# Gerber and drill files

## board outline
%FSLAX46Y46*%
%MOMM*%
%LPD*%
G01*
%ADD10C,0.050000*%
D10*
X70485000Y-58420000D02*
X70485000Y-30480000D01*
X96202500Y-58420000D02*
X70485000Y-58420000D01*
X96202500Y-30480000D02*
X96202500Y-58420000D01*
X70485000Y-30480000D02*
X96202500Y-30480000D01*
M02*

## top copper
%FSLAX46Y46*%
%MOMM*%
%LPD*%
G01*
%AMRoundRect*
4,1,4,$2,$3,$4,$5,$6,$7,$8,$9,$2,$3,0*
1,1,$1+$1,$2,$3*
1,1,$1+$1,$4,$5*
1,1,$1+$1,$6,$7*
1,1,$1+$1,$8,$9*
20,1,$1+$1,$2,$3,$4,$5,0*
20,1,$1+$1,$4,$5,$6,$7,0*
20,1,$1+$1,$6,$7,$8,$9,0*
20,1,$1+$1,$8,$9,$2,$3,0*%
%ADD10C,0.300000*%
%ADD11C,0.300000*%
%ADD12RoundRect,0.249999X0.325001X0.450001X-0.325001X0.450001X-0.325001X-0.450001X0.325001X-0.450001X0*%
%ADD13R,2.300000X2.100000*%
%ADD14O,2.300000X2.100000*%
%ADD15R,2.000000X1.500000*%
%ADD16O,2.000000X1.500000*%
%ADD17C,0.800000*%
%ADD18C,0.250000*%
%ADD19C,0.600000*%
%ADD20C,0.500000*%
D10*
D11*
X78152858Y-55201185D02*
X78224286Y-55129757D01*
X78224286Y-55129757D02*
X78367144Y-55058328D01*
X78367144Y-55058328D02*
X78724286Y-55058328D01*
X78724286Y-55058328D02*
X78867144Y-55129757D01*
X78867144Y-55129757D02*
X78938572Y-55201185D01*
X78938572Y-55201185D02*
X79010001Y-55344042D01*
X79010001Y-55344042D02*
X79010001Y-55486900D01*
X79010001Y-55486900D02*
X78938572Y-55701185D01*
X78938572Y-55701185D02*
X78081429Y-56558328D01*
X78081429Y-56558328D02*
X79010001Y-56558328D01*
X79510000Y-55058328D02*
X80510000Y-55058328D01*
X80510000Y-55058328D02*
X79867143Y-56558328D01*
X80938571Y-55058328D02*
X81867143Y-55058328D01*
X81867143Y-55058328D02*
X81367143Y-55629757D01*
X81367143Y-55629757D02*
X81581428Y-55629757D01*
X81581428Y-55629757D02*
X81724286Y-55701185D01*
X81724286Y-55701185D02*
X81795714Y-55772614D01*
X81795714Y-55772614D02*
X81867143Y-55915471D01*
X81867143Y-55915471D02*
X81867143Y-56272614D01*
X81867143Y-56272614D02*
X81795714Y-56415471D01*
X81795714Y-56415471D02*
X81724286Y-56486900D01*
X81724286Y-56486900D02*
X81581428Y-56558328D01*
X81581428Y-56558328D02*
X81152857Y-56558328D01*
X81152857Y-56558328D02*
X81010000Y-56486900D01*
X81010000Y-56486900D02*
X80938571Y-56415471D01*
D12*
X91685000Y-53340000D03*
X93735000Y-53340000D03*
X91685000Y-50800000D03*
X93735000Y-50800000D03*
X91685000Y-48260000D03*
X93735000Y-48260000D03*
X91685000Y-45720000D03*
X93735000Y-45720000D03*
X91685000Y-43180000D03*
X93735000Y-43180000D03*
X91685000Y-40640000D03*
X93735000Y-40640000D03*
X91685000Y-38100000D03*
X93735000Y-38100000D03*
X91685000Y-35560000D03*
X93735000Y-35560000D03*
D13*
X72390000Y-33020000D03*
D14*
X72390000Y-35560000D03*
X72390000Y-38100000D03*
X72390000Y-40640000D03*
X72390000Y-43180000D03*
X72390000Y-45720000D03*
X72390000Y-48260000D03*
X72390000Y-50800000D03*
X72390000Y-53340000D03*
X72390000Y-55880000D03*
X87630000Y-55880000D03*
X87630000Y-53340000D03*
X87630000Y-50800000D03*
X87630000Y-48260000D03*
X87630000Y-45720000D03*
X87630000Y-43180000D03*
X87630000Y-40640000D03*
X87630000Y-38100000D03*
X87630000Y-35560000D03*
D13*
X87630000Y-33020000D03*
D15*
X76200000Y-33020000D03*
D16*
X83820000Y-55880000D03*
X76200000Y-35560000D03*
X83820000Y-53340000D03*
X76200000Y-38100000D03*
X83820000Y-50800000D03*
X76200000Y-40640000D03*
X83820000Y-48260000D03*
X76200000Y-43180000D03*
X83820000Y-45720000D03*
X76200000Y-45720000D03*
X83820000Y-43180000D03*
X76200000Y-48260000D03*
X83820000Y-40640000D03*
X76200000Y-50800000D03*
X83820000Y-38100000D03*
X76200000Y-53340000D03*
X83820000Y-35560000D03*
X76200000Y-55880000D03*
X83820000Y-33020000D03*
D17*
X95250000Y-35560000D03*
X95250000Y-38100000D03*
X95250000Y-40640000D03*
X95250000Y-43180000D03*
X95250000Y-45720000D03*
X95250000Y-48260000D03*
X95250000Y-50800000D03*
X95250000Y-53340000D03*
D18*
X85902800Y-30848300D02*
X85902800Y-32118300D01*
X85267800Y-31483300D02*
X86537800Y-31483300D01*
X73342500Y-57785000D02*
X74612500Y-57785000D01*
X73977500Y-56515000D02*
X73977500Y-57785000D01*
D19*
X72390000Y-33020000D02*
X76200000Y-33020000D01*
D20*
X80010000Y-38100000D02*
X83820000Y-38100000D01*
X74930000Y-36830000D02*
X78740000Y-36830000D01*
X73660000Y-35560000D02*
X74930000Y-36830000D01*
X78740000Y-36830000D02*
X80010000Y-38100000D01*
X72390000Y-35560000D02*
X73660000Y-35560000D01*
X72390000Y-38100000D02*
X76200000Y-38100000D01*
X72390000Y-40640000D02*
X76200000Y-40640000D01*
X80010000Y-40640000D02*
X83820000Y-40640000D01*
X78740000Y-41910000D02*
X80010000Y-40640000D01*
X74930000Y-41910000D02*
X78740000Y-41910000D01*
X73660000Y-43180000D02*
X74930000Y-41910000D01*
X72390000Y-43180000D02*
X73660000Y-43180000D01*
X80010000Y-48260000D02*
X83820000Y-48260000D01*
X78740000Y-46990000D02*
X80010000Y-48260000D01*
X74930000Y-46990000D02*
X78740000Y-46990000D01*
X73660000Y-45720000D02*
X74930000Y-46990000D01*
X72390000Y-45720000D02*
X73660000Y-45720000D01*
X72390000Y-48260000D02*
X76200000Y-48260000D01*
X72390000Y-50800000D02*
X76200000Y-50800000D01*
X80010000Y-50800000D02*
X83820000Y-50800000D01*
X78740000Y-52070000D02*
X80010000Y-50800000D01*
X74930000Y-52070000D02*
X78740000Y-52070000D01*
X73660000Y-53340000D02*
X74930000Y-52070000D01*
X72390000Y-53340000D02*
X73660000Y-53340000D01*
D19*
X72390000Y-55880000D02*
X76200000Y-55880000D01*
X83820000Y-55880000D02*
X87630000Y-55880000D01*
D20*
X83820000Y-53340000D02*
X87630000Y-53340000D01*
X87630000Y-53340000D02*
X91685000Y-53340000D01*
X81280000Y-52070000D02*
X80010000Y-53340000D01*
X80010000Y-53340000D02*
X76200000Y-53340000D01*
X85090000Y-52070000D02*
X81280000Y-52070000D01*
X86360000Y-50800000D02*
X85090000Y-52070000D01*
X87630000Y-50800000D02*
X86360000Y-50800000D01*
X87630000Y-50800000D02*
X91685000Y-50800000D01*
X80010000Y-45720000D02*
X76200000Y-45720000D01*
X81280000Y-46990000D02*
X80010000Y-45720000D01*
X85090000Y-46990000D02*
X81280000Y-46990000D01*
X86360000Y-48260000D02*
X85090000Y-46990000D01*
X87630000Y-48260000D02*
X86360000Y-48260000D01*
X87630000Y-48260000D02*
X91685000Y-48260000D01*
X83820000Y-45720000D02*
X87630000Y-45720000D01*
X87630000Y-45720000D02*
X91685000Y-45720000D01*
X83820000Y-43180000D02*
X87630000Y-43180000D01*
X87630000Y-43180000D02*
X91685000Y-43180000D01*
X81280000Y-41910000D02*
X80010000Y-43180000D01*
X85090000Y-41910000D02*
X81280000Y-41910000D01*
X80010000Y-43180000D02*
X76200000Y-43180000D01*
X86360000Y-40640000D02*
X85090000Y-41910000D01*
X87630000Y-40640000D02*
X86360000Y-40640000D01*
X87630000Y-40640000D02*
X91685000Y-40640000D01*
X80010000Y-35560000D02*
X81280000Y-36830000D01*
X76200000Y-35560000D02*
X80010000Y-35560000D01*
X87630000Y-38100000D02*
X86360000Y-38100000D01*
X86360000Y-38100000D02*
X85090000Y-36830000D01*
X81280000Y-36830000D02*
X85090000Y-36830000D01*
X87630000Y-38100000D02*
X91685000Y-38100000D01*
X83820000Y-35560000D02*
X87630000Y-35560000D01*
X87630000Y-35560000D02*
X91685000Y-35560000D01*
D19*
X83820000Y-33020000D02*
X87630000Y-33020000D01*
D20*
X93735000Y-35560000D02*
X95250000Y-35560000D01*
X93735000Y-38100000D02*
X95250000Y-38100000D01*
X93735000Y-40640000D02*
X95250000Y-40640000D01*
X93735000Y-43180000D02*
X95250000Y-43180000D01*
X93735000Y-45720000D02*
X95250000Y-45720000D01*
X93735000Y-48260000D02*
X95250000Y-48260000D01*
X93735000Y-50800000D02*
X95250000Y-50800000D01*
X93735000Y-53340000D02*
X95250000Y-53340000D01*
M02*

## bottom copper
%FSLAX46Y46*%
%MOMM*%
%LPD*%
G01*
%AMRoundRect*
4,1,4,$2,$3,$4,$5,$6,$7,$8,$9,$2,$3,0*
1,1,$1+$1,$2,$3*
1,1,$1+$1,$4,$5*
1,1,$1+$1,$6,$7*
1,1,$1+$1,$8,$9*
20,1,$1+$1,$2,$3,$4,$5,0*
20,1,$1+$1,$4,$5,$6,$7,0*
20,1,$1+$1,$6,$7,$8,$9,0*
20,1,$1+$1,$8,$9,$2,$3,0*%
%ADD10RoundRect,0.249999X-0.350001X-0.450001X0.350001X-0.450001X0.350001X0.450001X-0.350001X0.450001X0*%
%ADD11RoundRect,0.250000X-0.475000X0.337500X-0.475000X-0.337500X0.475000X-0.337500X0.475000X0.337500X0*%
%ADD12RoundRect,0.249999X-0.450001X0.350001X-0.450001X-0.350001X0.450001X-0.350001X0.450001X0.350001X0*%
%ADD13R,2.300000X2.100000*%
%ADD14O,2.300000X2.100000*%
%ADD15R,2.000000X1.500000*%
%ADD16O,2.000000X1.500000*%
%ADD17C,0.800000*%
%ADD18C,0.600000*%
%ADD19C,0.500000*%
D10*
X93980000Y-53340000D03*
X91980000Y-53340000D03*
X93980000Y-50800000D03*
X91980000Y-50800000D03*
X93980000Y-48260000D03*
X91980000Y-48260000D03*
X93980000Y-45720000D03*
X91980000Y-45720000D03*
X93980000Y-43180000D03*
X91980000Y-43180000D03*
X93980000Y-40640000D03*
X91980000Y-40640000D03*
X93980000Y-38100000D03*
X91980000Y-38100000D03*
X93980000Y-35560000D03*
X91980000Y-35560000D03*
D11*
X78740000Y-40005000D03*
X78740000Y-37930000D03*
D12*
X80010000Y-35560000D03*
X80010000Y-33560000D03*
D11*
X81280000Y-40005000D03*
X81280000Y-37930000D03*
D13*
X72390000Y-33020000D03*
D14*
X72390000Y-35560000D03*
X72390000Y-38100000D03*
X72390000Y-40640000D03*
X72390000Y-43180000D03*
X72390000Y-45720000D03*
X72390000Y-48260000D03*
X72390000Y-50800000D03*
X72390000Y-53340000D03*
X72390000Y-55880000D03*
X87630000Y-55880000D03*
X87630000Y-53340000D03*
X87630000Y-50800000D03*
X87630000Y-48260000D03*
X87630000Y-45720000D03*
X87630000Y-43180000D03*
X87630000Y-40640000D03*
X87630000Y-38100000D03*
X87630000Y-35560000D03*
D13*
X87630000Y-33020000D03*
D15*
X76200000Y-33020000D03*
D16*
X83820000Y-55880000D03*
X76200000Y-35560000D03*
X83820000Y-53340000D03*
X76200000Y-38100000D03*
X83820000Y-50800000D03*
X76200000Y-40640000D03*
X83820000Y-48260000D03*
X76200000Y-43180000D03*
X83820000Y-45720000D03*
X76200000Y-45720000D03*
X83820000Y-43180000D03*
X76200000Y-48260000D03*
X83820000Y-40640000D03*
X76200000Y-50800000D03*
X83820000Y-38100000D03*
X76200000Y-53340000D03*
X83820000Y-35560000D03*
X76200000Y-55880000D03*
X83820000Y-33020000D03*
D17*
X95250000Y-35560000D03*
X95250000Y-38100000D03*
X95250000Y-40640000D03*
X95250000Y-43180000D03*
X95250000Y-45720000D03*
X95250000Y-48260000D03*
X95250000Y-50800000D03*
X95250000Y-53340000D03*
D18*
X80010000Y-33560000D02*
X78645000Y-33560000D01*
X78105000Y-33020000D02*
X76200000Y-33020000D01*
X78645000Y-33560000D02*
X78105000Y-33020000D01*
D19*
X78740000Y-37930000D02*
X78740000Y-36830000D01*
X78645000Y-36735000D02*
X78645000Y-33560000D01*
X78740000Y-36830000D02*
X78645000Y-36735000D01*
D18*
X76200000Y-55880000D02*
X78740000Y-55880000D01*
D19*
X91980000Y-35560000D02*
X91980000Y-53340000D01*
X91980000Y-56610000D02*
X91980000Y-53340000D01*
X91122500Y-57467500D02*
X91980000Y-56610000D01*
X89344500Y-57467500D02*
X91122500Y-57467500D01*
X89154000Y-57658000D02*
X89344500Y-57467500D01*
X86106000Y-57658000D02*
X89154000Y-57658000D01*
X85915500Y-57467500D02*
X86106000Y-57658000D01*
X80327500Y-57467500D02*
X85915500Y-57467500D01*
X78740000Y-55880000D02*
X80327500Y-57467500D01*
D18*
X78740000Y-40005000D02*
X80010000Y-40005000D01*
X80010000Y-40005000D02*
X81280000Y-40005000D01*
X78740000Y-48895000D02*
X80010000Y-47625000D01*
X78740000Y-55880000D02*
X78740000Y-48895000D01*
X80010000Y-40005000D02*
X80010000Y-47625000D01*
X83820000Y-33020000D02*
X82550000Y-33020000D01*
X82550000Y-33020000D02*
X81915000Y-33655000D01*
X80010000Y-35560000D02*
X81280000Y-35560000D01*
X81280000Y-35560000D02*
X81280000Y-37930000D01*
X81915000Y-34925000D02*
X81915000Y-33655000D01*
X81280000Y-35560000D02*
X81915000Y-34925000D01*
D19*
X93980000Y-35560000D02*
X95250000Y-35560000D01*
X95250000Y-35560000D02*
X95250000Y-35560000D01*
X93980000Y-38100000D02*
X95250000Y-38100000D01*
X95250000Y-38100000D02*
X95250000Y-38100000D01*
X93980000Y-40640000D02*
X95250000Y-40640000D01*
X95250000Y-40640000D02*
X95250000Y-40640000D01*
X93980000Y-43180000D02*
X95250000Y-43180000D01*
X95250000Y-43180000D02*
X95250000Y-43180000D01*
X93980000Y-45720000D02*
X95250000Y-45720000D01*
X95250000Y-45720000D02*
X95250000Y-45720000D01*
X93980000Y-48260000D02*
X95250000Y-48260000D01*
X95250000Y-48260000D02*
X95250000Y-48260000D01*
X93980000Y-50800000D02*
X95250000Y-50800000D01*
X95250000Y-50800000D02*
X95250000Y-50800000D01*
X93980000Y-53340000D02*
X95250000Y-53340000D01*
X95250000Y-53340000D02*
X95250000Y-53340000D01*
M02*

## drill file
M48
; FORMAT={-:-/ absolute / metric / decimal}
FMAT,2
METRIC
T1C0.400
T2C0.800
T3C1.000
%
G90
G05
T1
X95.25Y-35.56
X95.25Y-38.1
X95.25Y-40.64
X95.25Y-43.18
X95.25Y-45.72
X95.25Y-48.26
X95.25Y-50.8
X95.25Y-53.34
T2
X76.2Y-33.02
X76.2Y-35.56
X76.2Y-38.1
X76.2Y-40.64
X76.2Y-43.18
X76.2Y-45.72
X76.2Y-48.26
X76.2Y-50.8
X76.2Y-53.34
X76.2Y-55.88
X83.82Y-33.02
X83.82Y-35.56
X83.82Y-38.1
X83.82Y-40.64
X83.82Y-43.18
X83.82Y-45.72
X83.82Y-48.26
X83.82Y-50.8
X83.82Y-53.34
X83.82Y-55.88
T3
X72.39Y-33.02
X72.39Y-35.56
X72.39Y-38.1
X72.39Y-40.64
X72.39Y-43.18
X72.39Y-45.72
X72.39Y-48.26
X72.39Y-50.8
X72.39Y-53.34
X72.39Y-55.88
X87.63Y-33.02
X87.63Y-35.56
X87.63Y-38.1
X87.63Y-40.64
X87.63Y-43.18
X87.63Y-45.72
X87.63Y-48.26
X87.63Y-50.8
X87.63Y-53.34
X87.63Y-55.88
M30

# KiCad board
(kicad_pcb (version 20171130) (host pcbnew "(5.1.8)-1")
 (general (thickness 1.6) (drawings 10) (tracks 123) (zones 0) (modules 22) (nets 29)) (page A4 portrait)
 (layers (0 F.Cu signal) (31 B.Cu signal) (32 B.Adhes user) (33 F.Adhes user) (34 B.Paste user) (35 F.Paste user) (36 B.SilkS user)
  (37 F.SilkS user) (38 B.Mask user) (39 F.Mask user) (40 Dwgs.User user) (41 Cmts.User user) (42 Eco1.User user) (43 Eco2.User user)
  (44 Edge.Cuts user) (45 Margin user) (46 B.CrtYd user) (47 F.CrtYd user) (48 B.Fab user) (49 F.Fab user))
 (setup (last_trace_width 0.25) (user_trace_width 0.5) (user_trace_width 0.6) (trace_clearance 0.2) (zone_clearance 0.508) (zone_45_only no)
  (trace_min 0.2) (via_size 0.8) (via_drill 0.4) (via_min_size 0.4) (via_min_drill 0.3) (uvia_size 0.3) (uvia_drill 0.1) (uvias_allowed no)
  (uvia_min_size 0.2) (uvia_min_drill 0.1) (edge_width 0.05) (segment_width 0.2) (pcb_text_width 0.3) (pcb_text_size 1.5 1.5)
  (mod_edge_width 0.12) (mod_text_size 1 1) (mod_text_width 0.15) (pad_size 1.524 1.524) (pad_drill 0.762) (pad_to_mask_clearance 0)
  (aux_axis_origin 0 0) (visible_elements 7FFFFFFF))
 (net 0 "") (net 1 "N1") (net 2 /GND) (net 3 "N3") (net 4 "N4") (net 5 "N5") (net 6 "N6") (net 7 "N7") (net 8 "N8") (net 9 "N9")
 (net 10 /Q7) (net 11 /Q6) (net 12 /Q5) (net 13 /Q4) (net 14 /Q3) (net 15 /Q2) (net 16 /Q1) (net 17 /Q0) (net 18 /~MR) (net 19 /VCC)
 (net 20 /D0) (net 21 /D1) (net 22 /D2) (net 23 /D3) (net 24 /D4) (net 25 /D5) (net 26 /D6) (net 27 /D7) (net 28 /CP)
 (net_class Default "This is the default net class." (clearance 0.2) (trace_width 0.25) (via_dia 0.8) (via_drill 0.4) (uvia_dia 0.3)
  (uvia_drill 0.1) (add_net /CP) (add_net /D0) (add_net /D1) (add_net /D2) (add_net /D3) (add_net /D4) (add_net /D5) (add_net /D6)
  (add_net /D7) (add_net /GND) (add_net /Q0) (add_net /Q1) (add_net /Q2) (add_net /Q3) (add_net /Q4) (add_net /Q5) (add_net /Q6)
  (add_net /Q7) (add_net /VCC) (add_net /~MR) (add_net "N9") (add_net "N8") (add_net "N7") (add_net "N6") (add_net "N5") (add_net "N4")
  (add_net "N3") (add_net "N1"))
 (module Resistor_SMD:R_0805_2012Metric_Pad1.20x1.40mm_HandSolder (layer B.Cu) (at 92.98 53.34)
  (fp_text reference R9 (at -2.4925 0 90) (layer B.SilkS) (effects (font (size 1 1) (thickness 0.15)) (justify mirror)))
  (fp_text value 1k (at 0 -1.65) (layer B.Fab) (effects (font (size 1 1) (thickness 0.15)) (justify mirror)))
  (pad 2 smd roundrect (at 1 0) (size 1.2 1.4) (layers B.Cu B.Paste B.Mask) (roundrect_rratio 0.2083325) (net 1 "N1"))
  (pad 1 smd roundrect (at -1 0) (size 1.2 1.4) (layers B.Cu B.Paste B.Mask) (roundrect_rratio 0.2083325) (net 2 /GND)))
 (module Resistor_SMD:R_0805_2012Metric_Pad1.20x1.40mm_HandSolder (layer B.Cu) (at 92.98 50.8)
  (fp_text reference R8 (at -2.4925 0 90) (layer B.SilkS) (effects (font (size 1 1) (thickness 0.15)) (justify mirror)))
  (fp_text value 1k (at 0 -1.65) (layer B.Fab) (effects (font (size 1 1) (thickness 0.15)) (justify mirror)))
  (pad 2 smd roundrect (at 1 0) (size 1.2 1.4) (layers B.Cu B.Paste B.Mask) (roundrect_rratio 0.2083325) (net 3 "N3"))
  (pad 1 smd roundrect (at -1 0) (size 1.2 1.4) (layers B.Cu B.Paste B.Mask) (roundrect_rratio 0.2083325) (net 2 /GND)))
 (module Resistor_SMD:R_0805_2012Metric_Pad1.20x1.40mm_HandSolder (layer B.Cu) (at 92.98 48.26)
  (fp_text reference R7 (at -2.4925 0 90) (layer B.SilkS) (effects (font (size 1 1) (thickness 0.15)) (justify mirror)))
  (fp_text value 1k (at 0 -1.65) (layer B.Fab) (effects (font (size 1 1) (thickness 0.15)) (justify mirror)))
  (pad 2 smd roundrect (at 1 0) (size 1.2 1.4) (layers B.Cu B.Paste B.Mask) (roundrect_rratio 0.2083325) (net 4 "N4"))
  (pad 1 smd roundrect (at -1 0) (size 1.2 1.4) (layers B.Cu B.Paste B.Mask) (roundrect_rratio 0.2083325) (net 2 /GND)))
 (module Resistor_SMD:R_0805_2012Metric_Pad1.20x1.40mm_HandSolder (layer B.Cu) (at 92.98 45.72)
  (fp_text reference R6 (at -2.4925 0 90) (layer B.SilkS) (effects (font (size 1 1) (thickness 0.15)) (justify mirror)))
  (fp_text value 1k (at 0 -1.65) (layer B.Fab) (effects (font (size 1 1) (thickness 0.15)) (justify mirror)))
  (pad 2 smd roundrect (at 1 0) (size 1.2 1.4) (layers B.Cu B.Paste B.Mask) (roundrect_rratio 0.2083325) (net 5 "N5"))
  (pad 1 smd roundrect (at -1 0) (size 1.2 1.4) (layers B.Cu B.Paste B.Mask) (roundrect_rratio 0.2083325) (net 2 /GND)))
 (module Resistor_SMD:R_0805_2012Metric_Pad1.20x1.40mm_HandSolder (layer B.Cu) (at 92.98 43.18)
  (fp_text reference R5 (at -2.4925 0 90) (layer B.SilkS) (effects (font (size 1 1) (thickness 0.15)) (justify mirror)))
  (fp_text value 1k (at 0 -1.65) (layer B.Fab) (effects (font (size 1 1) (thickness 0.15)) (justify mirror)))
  (pad 2 smd roundrect (at 1 0) (size 1.2 1.4) (layers B.Cu B.Paste B.Mask) (roundrect_rratio 0.2083325) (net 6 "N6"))
  (pad 1 smd roundrect (at -1 0) (size 1.2 1.4) (layers B.Cu B.Paste B.Mask) (roundrect_rratio 0.2083325) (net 2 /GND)))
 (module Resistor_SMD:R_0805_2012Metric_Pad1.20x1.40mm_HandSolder (layer B.Cu) (at 92.98 40.64)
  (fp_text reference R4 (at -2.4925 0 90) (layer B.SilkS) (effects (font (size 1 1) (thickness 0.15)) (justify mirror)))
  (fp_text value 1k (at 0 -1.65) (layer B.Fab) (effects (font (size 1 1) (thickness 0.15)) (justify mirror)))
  (pad 2 smd roundrect (at 1 0) (size 1.2 1.4) (layers B.Cu B.Paste B.Mask) (roundrect_rratio 0.2083325) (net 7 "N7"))
  (pad 1 smd roundrect (at -1 0) (size 1.2 1.4) (layers B.Cu B.Paste B.Mask) (roundrect_rratio 0.2083325) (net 2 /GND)))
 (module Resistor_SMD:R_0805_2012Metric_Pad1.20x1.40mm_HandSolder (layer B.Cu) (at 92.98 38.1)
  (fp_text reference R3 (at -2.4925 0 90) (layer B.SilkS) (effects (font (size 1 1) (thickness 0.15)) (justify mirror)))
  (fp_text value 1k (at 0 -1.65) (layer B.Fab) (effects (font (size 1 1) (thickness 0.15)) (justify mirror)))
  (pad 2 smd roundrect (at 1 0) (size 1.2 1.4) (layers B.Cu B.Paste B.Mask) (roundrect_rratio 0.2083325) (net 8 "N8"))
  (pad 1 smd roundrect (at -1 0) (size 1.2 1.4) (layers B.Cu B.Paste B.Mask) (roundrect_rratio 0.2083325) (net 2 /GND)))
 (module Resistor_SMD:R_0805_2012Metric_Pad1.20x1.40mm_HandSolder (layer B.Cu) (at 92.98 35.56)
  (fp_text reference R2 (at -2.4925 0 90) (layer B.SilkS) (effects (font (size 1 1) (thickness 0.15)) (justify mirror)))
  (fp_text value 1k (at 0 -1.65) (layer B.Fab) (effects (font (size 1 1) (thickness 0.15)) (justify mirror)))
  (pad 2 smd roundrect (at 1 0) (size 1.2 1.4) (layers B.Cu B.Paste B.Mask) (roundrect_rratio 0.2083325) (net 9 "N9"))
  (pad 1 smd roundrect (at -1 0) (size 1.2 1.4) (layers B.Cu B.Paste B.Mask) (roundrect_rratio 0.2083325) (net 2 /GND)))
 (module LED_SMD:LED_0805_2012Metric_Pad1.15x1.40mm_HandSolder (layer F.Cu) (at 92.71 53.34 180)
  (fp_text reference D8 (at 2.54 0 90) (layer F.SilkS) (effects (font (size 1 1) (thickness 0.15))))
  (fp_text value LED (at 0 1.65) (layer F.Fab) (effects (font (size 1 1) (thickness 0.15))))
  (pad 2 smd roundrect (at 1.025 0 180) (size 1.15 1.4) (layers F.Cu F.Paste F.Mask) (roundrect_rratio 0.2173904347826087) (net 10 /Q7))
  (pad 1 smd roundrect (at -1.025 0 180) (size 1.15 1.4) (layers F.Cu F.Paste F.Mask) (roundrect_rratio 0.2173904347826087) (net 1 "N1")))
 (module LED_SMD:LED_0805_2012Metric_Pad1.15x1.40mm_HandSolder (layer F.Cu) (at 92.71 50.8 180)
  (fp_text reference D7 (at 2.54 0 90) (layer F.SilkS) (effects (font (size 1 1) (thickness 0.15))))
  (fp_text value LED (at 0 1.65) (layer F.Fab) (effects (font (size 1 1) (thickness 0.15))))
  (pad 2 smd roundrect (at 1.025 0 180) (size 1.15 1.4) (layers F.Cu F.Paste F.Mask) (roundrect_rratio 0.2173904347826087) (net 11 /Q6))
  (pad 1 smd roundrect (at -1.025 0 180) (size 1.15 1.4) (layers F.Cu F.Paste F.Mask) (roundrect_rratio 0.2173904347826087) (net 3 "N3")))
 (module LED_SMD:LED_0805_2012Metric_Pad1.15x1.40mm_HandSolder (layer F.Cu) (at 92.71 48.26 180)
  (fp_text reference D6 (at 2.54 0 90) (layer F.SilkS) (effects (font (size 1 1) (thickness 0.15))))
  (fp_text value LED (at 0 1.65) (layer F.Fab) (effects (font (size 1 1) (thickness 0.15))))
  (pad 2 smd roundrect (at 1.025 0 180) (size 1.15 1.4) (layers F.Cu F.Paste F.Mask) (roundrect_rratio 0.2173904347826087) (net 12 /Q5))
  (pad 1 smd roundrect (at -1.025 0 180) (size 1.15 1.4) (layers F.Cu F.Paste F.Mask) (roundrect_rratio 0.2173904347826087) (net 4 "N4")))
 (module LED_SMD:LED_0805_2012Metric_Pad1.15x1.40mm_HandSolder (layer F.Cu) (at 92.71 45.72 180)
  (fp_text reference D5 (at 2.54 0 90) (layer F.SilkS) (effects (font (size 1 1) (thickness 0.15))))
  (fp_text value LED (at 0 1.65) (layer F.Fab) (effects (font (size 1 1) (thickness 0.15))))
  (pad 2 smd roundrect (at 1.025 0 180) (size 1.15 1.4) (layers F.Cu F.Paste F.Mask) (roundrect_rratio 0.2173904347826087) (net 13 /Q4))
  (pad 1 smd roundrect (at -1.025 0 180) (size 1.15 1.4) (layers F.Cu F.Paste F.Mask) (roundrect_rratio 0.2173904347826087) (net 5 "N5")))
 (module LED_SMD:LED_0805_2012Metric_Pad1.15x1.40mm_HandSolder (layer F.Cu) (at 92.71 43.18 180)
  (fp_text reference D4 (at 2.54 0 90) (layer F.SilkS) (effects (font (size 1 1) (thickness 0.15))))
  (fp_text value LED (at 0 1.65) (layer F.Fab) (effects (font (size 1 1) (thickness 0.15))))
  (pad 2 smd roundrect (at 1.025 0 180) (size 1.15 1.4) (layers F.Cu F.Paste F.Mask) (roundrect_rratio 0.2173904347826087) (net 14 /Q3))
  (pad 1 smd roundrect (at -1.025 0 180) (size 1.15 1.4) (layers F.Cu F.Paste F.Mask) (roundrect_rratio 0.2173904347826087) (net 6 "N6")))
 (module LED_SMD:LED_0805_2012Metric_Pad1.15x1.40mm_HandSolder (layer F.Cu) (at 92.71 40.64 180)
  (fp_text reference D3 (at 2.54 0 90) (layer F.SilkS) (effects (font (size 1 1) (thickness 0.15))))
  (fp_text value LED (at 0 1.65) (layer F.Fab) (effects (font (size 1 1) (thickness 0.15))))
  (pad 2 smd roundrect (at 1.025 0 180) (size 1.15 1.4) (layers F.Cu F.Paste F.Mask) (roundrect_rratio 0.2173904347826087) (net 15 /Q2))
  (pad 1 smd roundrect (at -1.025 0 180) (size 1.15 1.4) (layers F.Cu F.Paste F.Mask) (roundrect_rratio 0.2173904347826087) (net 7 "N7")))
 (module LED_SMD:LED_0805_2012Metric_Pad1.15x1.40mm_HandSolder (layer F.Cu) (at 92.71 38.1 180)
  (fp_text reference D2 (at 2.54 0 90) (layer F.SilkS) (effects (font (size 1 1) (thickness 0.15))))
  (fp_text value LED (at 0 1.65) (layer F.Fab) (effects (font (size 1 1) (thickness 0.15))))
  (pad 2 smd roundrect (at 1.025 0 180) (size 1.15 1.4) (layers F.Cu F.Paste F.Mask) (roundrect_rratio 0.2173904347826087) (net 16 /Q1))
  (pad 1 smd roundrect (at -1.025 0 180) (size 1.15 1.4) (layers F.Cu F.Paste F.Mask) (roundrect_rratio 0.2173904347826087) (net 8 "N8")))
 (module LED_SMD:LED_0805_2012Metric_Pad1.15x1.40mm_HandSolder (layer F.Cu) (at 92.71 35.56 180)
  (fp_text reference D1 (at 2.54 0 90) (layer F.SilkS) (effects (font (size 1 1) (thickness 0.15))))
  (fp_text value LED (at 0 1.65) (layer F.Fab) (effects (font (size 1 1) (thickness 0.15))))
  (pad 2 smd roundrect (at 1.025 0 180) (size 1.15 1.4) (layers F.Cu F.Paste F.Mask) (roundrect_rratio 0.2173904347826087) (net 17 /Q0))
  (pad 1 smd roundrect (at -1.025 0 180) (size 1.15 1.4) (layers F.Cu F.Paste F.Mask) (roundrect_rratio 0.2173904347826087) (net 9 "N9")))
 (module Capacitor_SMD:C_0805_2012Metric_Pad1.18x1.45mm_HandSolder (layer B.Cu) (at 78.74 38.9675 270)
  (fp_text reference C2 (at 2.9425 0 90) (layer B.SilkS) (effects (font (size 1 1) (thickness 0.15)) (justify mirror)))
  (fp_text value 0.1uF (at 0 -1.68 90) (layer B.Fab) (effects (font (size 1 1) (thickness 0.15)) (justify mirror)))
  (pad 2 smd roundrect (at 1.0375 0 270) (size 1.175 1.45) (layers B.Cu B.Paste B.Mask) (roundrect_rratio 0.2127659574468085) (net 2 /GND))
  (pad 1 smd roundrect (at -1.0375 0 270) (size 1.175 1.45) (layers B.Cu B.Paste B.Mask) (roundrect_rratio 0.2127659574468085) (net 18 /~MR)))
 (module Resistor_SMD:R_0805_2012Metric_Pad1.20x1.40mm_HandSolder (layer B.Cu) (at 80.01 34.56 270)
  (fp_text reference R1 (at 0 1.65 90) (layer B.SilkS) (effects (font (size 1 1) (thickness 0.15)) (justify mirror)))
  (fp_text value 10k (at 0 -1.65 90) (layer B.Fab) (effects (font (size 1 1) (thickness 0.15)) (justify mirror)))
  (pad 2 smd roundrect (at 1 0 270) (size 1.2 1.4) (layers B.Cu B.Paste B.Mask) (roundrect_rratio 0.2083325) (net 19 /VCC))
  (pad 1 smd roundrect (at -1 0 270) (size 1.2 1.4) (layers B.Cu B.Paste B.Mask) (roundrect_rratio 0.2083325) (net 18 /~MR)))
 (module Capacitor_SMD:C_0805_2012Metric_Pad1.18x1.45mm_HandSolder (layer B.Cu) (at 81.28 38.9675 270)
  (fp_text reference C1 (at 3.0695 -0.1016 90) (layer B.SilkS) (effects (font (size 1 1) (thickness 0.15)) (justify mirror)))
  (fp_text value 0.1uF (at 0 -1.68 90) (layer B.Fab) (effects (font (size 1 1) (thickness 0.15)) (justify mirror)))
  (pad 2 smd roundrect (at 1.0375 0 270) (size 1.175 1.45) (layers B.Cu B.Paste B.Mask) (roundrect_rratio 0.2127659574468085) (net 2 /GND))
  (pad 1 smd roundrect (at -1.0375 0 270) (size 1.175 1.45) (layers B.Cu B.Paste B.Mask) (roundrect_rratio 0.2127659574468085) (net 19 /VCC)))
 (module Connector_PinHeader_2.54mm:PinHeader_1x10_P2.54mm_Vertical (layer B.Cu) (at 72.39 33.02 180)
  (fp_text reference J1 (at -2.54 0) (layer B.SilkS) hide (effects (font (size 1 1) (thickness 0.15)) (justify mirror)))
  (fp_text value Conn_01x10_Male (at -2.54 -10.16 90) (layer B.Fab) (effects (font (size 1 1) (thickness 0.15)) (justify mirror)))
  (pad 1 thru_hole rect (at 0 0 180) (size 2.3 2.1) (drill 1) (layers *.Cu *.Mask) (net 18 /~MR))
  (pad 2 thru_hole oval (at 0 -2.54 180) (size 2.3 2.1) (drill 1) (layers *.Cu *.Mask) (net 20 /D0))
  (pad 3 thru_hole oval (at 0 -5.08 180) (size 2.3 2.1) (drill 1) (layers *.Cu *.Mask) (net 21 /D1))
  (pad 4 thru_hole oval (at 0 -7.62 180) (size 2.3 2.1) (drill 1) (layers *.Cu *.Mask) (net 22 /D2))
  (pad 5 thru_hole oval (at 0 -10.16 180) (size 2.3 2.1) (drill 1) (layers *.Cu *.Mask) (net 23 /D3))
  (pad 6 thru_hole oval (at 0 -12.7 180) (size 2.3 2.1) (drill 1) (layers *.Cu *.Mask) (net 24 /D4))
  (pad 7 thru_hole oval (at 0 -15.24 180) (size 2.3 2.1) (drill 1) (layers *.Cu *.Mask) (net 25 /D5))
  (pad 8 thru_hole oval (at 0 -17.78 180) (size 2.3 2.1) (drill 1) (layers *.Cu *.Mask) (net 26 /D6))
  (pad 9 thru_hole oval (at 0 -20.32 180) (size 2.3 2.1) (drill 1) (layers *.Cu *.Mask) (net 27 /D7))
  (pad 10 thru_hole oval (at 0 -22.86 180) (size 2.3 2.1) (drill 1) (layers *.Cu *.Mask) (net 2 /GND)))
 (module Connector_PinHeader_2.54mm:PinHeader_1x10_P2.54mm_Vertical (layer B.Cu) (at 87.63 33.02 180)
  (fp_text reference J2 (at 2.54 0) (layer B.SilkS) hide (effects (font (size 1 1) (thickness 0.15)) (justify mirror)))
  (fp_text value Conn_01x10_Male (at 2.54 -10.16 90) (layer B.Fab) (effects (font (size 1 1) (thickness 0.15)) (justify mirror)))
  (pad 10 thru_hole oval (at 0 -22.86 180) (size 2.3 2.1) (drill 1) (layers *.Cu *.Mask) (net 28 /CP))
  (pad 9 thru_hole oval (at 0 -20.32 180) (size 2.3 2.1) (drill 1) (layers *.Cu *.Mask) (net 10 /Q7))
  (pad 8 thru_hole oval (at 0 -17.78 180) (size 2.3 2.1) (drill 1) (layers *.Cu *.Mask) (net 11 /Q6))
  (pad 7 thru_hole oval (at 0 -15.24 180) (size 2.3 2.1) (drill 1) (layers *.Cu *.Mask) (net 12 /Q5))
  (pad 6 thru_hole oval (at 0 -12.7 180) (size 2.3 2.1) (drill 1) (layers *.Cu *.Mask) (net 13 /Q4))
  (pad 5 thru_hole oval (at 0 -10.16 180) (size 2.3 2.1) (drill 1) (layers *.Cu *.Mask) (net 14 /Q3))
  (pad 4 thru_hole oval (at 0 -7.62 180) (size 2.3 2.1) (drill 1) (layers *.Cu *.Mask) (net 15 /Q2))
  (pad 3 thru_hole oval (at 0 -5.08 180) (size 2.3 2.1) (drill 1) (layers *.Cu *.Mask) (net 16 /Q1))
  (pad 2 thru_hole oval (at 0 -2.54 180) (size 2.3 2.1) (drill 1) (layers *.Cu *.Mask) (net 17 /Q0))
  (pad 1 thru_hole rect (at 0 0 180) (size 2.3 2.1) (drill 1) (layers *.Cu *.Mask) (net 19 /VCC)))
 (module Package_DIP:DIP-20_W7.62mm (layer F.Cu) (at 76.2 33.02)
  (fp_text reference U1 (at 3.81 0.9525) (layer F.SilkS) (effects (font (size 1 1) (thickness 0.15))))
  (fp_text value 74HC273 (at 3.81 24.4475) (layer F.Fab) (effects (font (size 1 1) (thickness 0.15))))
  (pad 1 thru_hole rect (at 0 0) (size 2 1.5) (drill 0.8) (layers *.Cu *.Mask) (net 18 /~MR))
  (pad 11 thru_hole oval (at 7.62 22.86) (size 2 1.5) (drill 0.8) (layers *.Cu *.Mask) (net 28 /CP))
  (pad 2 thru_hole oval (at 0 2.54) (size 2 1.5) (drill 0.8) (layers *.Cu *.Mask) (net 16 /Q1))
  (pad 12 thru_hole oval (at 7.62 20.32) (size 2 1.5) (drill 0.8) (layers *.Cu *.Mask) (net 10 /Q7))
  (pad 3 thru_hole oval (at 0 5.08) (size 2 1.5) (drill 0.8) (layers *.Cu *.Mask) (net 21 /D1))
  (pad 13 thru_hole oval (at 7.62 17.78) (size 2 1.5) (drill 0.8) (layers *.Cu *.Mask) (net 27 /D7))
  (pad 4 thru_hole oval (at 0 7.62) (size 2 1.5) (drill 0.8) (layers *.Cu *.Mask) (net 22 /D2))
  (pad 14 thru_hole oval (at 7.62 15.24) (size 2 1.5) (drill 0.8) (layers *.Cu *.Mask) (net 24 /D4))
  (pad 5 thru_hole oval (at 0 10.16) (size 2 1.5) (drill 0.8) (layers *.Cu *.Mask) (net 15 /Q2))
  (pad 15 thru_hole oval (at 7.62 12.7) (size 2 1.5) (drill 0.8) (layers *.Cu *.Mask) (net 13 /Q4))
  (pad 6 thru_hole oval (at 0 12.7) (size 2 1.5) (drill 0.8) (layers *.Cu *.Mask) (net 12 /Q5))
  (pad 16 thru_hole oval (at 7.62 10.16) (size 2 1.5) (drill 0.8) (layers *.Cu *.Mask) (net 14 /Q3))
  (pad 7 thru_hole oval (at 0 15.24) (size 2 1.5) (drill 0.8) (layers *.Cu *.Mask) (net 25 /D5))
  (pad 17 thru_hole oval (at 7.62 7.62) (size 2 1.5) (drill 0.8) (layers *.Cu *.Mask) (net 23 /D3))
  (pad 8 thru_hole oval (at 0 17.78) (size 2 1.5) (drill 0.8) (layers *.Cu *.Mask) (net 26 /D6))
  (pad 18 thru_hole oval (at 7.62 5.08) (size 2 1.5) (drill 0.8) (layers *.Cu *.Mask) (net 20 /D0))
  (pad 9 thru_hole oval (at 0 20.32) (size 2 1.5) (drill 0.8) (layers *.Cu *.Mask) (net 11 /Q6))
  (pad 19 thru_hole oval (at 7.62 2.54) (size 2 1.5) (drill 0.8) (layers *.Cu *.Mask) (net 17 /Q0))
  (pad 10 thru_hole oval (at 0 22.86) (size 2 1.5) (drill 0.8) (layers *.Cu *.Mask) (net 2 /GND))
  (pad 20 thru_hole oval (at 7.62 0) (size 2 1.5) (drill 0.8) (layers *.Cu *.Mask) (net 19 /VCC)))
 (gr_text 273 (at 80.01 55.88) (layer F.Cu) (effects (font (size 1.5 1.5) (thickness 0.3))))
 (gr_line (start 70.485 58.42) (end 70.485 30.48) (layer Edge.Cuts) (width 0.05))
 (gr_line (start 96.2025 58.42) (end 70.485 58.42) (layer Edge.Cuts) (width 0.05))
 (gr_line (start 96.2025 30.48) (end 96.2025 58.42) (layer Edge.Cuts) (width 0.05))
 (gr_line (start 70.485 30.48) (end 96.2025 30.48) (layer Edge.Cuts) (width 0.05))
 (segment (start 85.9028 30.8483) (end 85.9028 32.1183) (width 0.25) (layer F.Cu) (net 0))
 (segment (start 85.2678 31.4833) (end 86.5378 31.4833) (width 0.25) (layer F.Cu) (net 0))
 (segment (start 73.3425 57.785) (end 74.6125 57.785) (width 0.25) (layer F.Cu) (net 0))
 (segment (start 73.9775 56.515) (end 73.9775 57.785) (width 0.25) (layer F.Cu) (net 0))
 (segment (start 72.39 33.02) (end 76.2 33.02) (width 0.6) (layer F.Cu) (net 18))
 (segment (start 80.01 33.56) (end 78.645 33.56) (width 0.6) (layer B.Cu) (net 18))
 (segment (start 78.105 33.02) (end 76.2 33.02) (width 0.6) (layer B.Cu) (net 18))
 (segment (start 78.645 33.56) (end 78.105 33.02) (width 0.6) (layer B.Cu) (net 18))
 (segment (start 78.74 37.93) (end 78.74 36.83) (width 0.5) (layer B.Cu) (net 18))
 (segment (start 78.645 36.735) (end 78.645 33.56) (width 0.5) (layer B.Cu) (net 18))
 (segment (start 78.74 36.83) (end 78.645 36.735) (width 0.5) (layer B.Cu) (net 18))
 (segment (start 80.01 38.1) (end 83.82 38.1) (width 0.5) (layer F.Cu) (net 20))
 (segment (start 74.93 36.83) (end 78.74 36.83) (width 0.5) (layer F.Cu) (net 20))
 (segment (start 73.66 35.56) (end 74.93 36.83) (width 0.5) (layer F.Cu) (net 20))
 (segment (start 78.74 36.83) (end 80.01 38.1) (width 0.5) (layer F.Cu) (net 20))
 (segment (start 72.39 35.56) (end 73.66 35.56) (width 0.5) (layer F.Cu) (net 20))
 (segment (start 72.39 38.1) (end 76.2 38.1) (width 0.5) (layer F.Cu) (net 21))
 (segment (start 72.39 40.64) (end 76.2 40.64) (width 0.5) (layer F.Cu) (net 22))
 (segment (start 80.01 40.64) (end 83.82 40.64) (width 0.5) (layer F.Cu) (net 23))
 (segment (start 78.74 41.91) (end 80.01 40.64) (width 0.5) (layer F.Cu) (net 23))
 (segment (start 74.93 41.91) (end 78.74 41.91) (width 0.5) (layer F.Cu) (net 23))
 (segment (start 73.66 43.18) (end 74.93 41.91) (width 0.5) (layer F.Cu) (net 23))
 (segment (start 72.39 43.18) (end 73.66 43.18) (width 0.5) (layer F.Cu) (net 23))
 (segment (start 80.01 48.26) (end 83.82 48.26) (width 0.5) (layer F.Cu) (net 24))
 (segment (start 78.74 46.99) (end 80.01 48.26) (width 0.5) (layer F.Cu) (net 24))
 (segment (start 74.93 46.99) (end 78.74 46.99) (width 0.5) (layer F.Cu) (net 24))
 (segment (start 73.66 45.72) (end 74.93 46.99) (width 0.5) (layer F.Cu) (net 24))
 (segment (start 72.39 45.72) (end 73.66 45.72) (width 0.5) (layer F.Cu) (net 24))
 (segment (start 72.39 48.26) (end 76.2 48.26) (width 0.5) (layer F.Cu) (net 25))
 (segment (start 72.39 50.8) (end 76.2 50.8) (width 0.5) (layer F.Cu) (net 26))
 (segment (start 80.01 50.8) (end 83.82 50.8) (width 0.5) (layer F.Cu) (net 27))
 (segment (start 78.74 52.07) (end 80.01 50.8) (width 0.5) (layer F.Cu) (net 27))
 (segment (start 74.93 52.07) (end 78.74 52.07) (width 0.5) (layer F.Cu) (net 27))
 (segment (start 73.66 53.34) (end 74.93 52.07) (width 0.5) (layer F.Cu) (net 27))
 (segment (start 72.39 53.34) (end 73.66 53.34) (width 0.5) (layer F.Cu) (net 27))
 (segment (start 72.39 55.88) (end 76.2 55.88) (width 0.6) (layer F.Cu) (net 2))
 (segment (start 76.2 55.88) (end 78.74 55.88) (width 0.6) (layer B.Cu) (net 2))
 (segment (start 91.98 35.56) (end 91.98 53.34) (width 0.5) (layer B.Cu) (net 2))
 (segment (start 91.98 56.61) (end 91.98 53.34) (width 0.5) (layer B.Cu) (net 2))
 (segment (start 91.1225 57.4675) (end 91.98 56.61) (width 0.5) (layer B.Cu) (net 2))
 (segment (start 89.3445 57.4675) (end 91.1225 57.4675) (width 0.5) (layer B.Cu) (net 2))
 (segment (start 89.154 57.658) (end 89.3445 57.4675) (width 0.5) (layer B.Cu) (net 2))
 (segment (start 86.106 57.658) (end 89.154 57.658) (width 0.5) (layer B.Cu) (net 2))
 (segment (start 85.9155 57.4675) (end 86.106 57.658) (width 0.5) (layer B.Cu) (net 2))
 (segment (start 80.3275 57.4675) (end 85.9155 57.4675) (width 0.5) (layer B.Cu) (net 2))
 (segment (start 78.74 55.88) (end 80.3275 57.4675) (width 0.5) (layer B.Cu) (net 2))
 (segment (start 78.74 40.005) (end 80.01 40.005) (width 0.6) (layer B.Cu) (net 2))
 (segment (start 80.01 40.005) (end 81.28 40.005) (width 0.6) (layer B.Cu) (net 2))
 (segment (start 78.74 48.895) (end 80.01 47.625) (width 0.6) (layer B.Cu) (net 2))
 (segment (start 78.74 55.88) (end 78.74 48.895) (width 0.6) (layer B.Cu) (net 2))
 (segment (start 80.01 40.005) (end 80.01 47.625) (width 0.6) (layer B.Cu) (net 2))
 (segment (start 83.82 55.88) (end 87.63 55.88) (width 0.6) (layer F.Cu) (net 28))
 (segment (start 83.82 53.34) (end 87.63 53.34) (width 0.5) (layer F.Cu) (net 10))
 (segment (start 87.63 53.34) (end 91.685 53.34) (width 0.5) (layer F.Cu) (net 10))
 (segment (start 81.28 52.07) (end 80.01 53.34) (width 0.5) (layer F.Cu) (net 11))
 (segment (start 80.01 53.34) (end 76.2 53.34) (width 0.5) (layer F.Cu) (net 11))
 (segment (start 85.09 52.07) (end 81.28 52.07) (width 0.5) (layer F.Cu) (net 11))
 (segment (start 86.36 50.8) (end 85.09 52.07) (width 0.5) (layer F.Cu) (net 11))
 (segment (start 87.63 50.8) (end 86.36 50.8) (width 0.5) (layer F.Cu) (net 11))
 (segment (start 87.63 50.8) (end 91.685 50.8) (width 0.5) (layer F.Cu) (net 11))
 (segment (start 80.01 45.72) (end 76.2 45.72) (width 0.5) (layer F.Cu) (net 12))
 (segment (start 81.28 46.99) (end 80.01 45.72) (width 0.5) (layer F.Cu) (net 12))
 (segment (start 85.09 46.99) (end 81.28 46.99) (width 0.5) (layer F.Cu) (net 12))
 (segment (start 86.36 48.26) (end 85.09 46.99) (width 0.5) (layer F.Cu) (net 12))
 (segment (start 87.63 48.26) (end 86.36 48.26) (width 0.5) (layer F.Cu) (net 12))
 (segment (start 87.63 48.26) (end 91.685 48.26) (width 0.5) (layer F.Cu) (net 12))
 (segment (start 83.82 45.72) (end 87.63 45.72) (width 0.5) (layer F.Cu) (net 13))
 (segment (start 87.63 45.72) (end 91.685 45.72) (width 0.5) (layer F.Cu) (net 13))
 (segment (start 83.82 43.18) (end 87.63 43.18) (width 0.5) (layer F.Cu) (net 14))
 (segment (start 87.63 43.18) (end 91.685 43.18) (width 0.5) (layer F.Cu) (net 14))
 (segment (start 81.28 41.91) (end 80.01 43.18) (width 0.5) (layer F.Cu) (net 15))
 (segment (start 85.09 41.91) (end 81.28 41.91) (width 0.5) (layer F.Cu) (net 15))
 (segment (start 80.01 43.18) (end 76.2 43.18) (width 0.5) (layer F.Cu) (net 15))
 (segment (start 86.36 40.64) (end 85.09 41.91) (width 0.5) (layer F.Cu) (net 15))
 (segment (start 87.63 40.64) (end 86.36 40.64) (width 0.5) (layer F.Cu) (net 15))
 (segment (start 87.63 40.64) (end 91.685 40.64) (width 0.5) (layer F.Cu) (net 15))
 (segment (start 80.01 35.56) (end 81.28 36.83) (width 0.5) (layer F.Cu) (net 16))
 (segment (start 76.2 35.56) (end 80.01 35.56) (width 0.5) (layer F.Cu) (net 16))
 (segment (start 87.63 38.1) (end 86.36 38.1) (width 0.5) (layer F.Cu) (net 16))
 (segment (start 86.36 38.1) (end 85.09 36.83) (width 0.5) (layer F.Cu) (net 16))
 (segment (start 81.28 36.83) (end 85.09 36.83) (width 0.5) (layer F.Cu) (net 16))
 (segment (start 87.63 38.1) (end 91.685 38.1) (width 0.5) (layer F.Cu) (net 16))
 (segment (start 83.82 35.56) (end 87.63 35.56) (width 0.5) (layer F.Cu) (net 17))
 (segment (start 87.63 35.56) (end 91.685 35.56) (width 0.5) (layer F.Cu) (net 17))
 (segment (start 83.82 33.02) (end 87.63 33.02) (width 0.6) (layer F.Cu) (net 19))
 (segment (start 83.82 33.02) (end 82.55 33.02) (width 0.6) (layer B.Cu) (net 19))
 (segment (start 82.55 33.02) (end 81.915 33.655) (width 0.6) (layer B.Cu) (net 19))
 (segment (start 80.01 35.56) (end 81.28 35.56) (width 0.6) (layer B.Cu) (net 19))
 (segment (start 81.28 35.56) (end 81.28 37.93) (width 0.6) (layer B.Cu) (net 19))
 (segment (start 81.915 34.925) (end 81.915 33.655) (width 0.6) (layer B.Cu) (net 19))
 (segment (start 81.28 35.56) (end 81.915 34.925) (width 0.6) (layer B.Cu) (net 19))
 (segment (start 93.98 35.56) (end 95.25 35.56) (width 0.5) (layer B.Cu) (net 9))
 (segment (start 95.25 35.56) (end 95.25 35.56) (width 0.5) (layer B.Cu) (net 9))
 (via (at 95.25 35.56) (size 0.8) (drill 0.4) (layers F.Cu B.Cu) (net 9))
 (segment (start 93.735 35.56) (end 95.25 35.56) (width 0.5) (layer F.Cu) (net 9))
 (segment (start 93.98 38.1) (end 95.25 38.1) (width 0.5) (layer B.Cu) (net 8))
 (segment (start 95.25 38.1) (end 95.25 38.1) (width 0.5) (layer B.Cu) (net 8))
 (via (at 95.25 38.1) (size 0.8) (drill 0.4) (layers F.Cu B.Cu) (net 8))
 (segment (start 93.735 38.1) (end 95.25 38.1) (width 0.5) (layer F.Cu) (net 8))
 (segment (start 93.98 40.64) (end 95.25 40.64) (width 0.5) (layer B.Cu) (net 7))
 (segment (start 95.25 40.64) (end 95.25 40.64) (width 0.5) (layer B.Cu) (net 7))
 (via (at 95.25 40.64) (size 0.8) (drill 0.4) (layers F.Cu B.Cu) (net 7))
 (segment (start 93.735 40.64) (end 95.25 40.64) (width 0.5) (layer F.Cu) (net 7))
 (segment (start 93.98 43.18) (end 95.25 43.18) (width 0.5) (layer B.Cu) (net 6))
 (segment (start 95.25 43.18) (end 95.25 43.18) (width 0.5) (layer B.Cu) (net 6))
 (via (at 95.25 43.18) (size 0.8) (drill 0.4) (layers F.Cu B.Cu) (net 6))
 (segment (start 93.735 43.18) (end 95.25 43.18) (width 0.5) (layer F.Cu) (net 6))
 (segment (start 93.98 45.72) (end 95.25 45.72) (width 0.5) (layer B.Cu) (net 5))
 (segment (start 95.25 45.72) (end 95.25 45.72) (width 0.5) (layer B.Cu) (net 5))
 (via (at 95.25 45.72) (size 0.8) (drill 0.4) (layers F.Cu B.Cu) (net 5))
 (segment (start 93.735 45.72) (end 95.25 45.72) (width 0.5) (layer F.Cu) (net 5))
 (segment (start 93.98 48.26) (end 95.25 48.26) (width 0.5) (layer B.Cu) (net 4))
 (segment (start 95.25 48.26) (end 95.25 48.26) (width 0.5) (layer B.Cu) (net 4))
 (via (at 95.25 48.26) (size 0.8) (drill 0.4) (layers F.Cu B.Cu) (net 4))
 (segment (start 93.735 48.26) (end 95.25 48.26) (width 0.5) (layer F.Cu) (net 4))
 (segment (start 93.98 50.8) (end 95.25 50.8) (width 0.5) (layer B.Cu) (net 3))
 (segment (start 95.25 50.8) (end 95.25 50.8) (width 0.5) (layer B.Cu) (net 3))
 (via (at 95.25 50.8) (size 0.8) (drill 0.4) (layers F.Cu B.Cu) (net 3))
 (segment (start 93.735 50.8) (end 95.25 50.8) (width 0.5) (layer F.Cu) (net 3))
 (segment (start 93.98 53.34) (end 95.25 53.34) (width 0.5) (layer B.Cu) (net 1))
 (segment (start 95.25 53.34) (end 95.25 53.34) (width 0.5) (layer B.Cu) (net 1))
 (via (at 95.25 53.34) (size 0.8) (drill 0.4) (layers F.Cu B.Cu) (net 1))
 (segment (start 93.735 53.34) (end 95.25 53.34) (width 0.5) (layer F.Cu) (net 1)))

